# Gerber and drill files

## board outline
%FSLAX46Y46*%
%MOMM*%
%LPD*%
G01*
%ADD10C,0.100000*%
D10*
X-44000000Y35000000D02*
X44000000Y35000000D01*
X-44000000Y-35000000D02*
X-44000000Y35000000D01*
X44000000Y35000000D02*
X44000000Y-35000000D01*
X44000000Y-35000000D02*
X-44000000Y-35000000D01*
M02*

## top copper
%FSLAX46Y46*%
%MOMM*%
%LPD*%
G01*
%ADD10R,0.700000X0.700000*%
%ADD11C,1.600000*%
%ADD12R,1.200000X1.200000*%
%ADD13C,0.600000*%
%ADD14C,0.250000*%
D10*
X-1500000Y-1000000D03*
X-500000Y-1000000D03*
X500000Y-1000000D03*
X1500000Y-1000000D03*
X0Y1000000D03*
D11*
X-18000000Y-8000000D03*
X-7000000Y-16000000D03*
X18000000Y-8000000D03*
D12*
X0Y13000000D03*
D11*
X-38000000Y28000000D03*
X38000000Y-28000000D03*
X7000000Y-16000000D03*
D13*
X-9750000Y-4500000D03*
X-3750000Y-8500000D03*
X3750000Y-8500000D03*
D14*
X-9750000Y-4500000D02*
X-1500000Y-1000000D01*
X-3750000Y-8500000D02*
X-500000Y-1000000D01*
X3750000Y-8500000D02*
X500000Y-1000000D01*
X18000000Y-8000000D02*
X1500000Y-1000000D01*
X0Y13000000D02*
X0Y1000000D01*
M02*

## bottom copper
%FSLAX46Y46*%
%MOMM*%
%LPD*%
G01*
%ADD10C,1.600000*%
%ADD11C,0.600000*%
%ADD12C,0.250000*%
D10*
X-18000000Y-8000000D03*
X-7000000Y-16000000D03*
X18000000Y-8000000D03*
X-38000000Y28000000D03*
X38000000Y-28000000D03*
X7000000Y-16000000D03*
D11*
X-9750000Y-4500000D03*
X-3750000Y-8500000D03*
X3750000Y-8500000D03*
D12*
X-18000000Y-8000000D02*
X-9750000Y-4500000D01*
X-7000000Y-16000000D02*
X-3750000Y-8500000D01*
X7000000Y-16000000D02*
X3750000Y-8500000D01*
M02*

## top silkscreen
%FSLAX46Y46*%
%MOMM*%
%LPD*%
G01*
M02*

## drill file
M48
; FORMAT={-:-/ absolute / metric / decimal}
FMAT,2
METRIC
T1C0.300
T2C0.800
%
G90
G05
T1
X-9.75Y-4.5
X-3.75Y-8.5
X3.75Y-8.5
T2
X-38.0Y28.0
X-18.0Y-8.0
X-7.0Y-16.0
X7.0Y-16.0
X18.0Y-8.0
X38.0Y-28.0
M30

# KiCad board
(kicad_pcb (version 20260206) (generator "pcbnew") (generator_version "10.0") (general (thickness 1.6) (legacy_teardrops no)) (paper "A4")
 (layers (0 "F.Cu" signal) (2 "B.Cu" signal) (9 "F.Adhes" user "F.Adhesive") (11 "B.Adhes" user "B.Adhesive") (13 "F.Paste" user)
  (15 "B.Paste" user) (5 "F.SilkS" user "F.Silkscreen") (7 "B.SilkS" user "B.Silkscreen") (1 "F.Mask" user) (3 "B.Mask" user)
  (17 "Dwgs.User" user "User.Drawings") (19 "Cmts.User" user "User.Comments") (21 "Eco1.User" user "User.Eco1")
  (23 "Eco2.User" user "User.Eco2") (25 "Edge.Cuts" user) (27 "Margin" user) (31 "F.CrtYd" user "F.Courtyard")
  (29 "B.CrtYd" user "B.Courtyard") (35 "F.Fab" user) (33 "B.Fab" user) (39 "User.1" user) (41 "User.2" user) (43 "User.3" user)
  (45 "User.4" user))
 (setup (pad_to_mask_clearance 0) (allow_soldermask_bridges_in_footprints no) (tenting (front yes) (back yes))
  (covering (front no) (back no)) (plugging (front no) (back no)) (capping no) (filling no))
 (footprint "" (layer "F.Cu") (at 0 0)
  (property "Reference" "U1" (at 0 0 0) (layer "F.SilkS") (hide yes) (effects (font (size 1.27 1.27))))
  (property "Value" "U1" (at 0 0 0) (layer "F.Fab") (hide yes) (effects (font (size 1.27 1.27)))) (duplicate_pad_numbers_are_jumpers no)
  (pad "1" smd rect (at -1.5 1) (size 0.7 0.7) (layers "F.Cu" "F.Mask" "F.Paste") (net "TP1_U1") (thermal_bridge_angle 45))
  (pad "2" smd rect (at -0.5 1) (size 0.7 0.7) (layers "F.Cu" "F.Mask" "F.Paste") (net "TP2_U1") (thermal_bridge_angle 45))
  (pad "3" smd rect (at 0.5 1) (size 0.7 0.7) (layers "F.Cu" "F.Mask" "F.Paste") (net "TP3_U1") (thermal_bridge_angle 45))
  (pad "4" smd rect (at 1.5 1) (size 0.7 0.7) (layers "F.Cu" "F.Mask" "F.Paste") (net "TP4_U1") (thermal_bridge_angle 45))
  (pad "5" smd rect (at 0 -1) (size 0.7 0.7) (layers "F.Cu" "F.Mask" "F.Paste") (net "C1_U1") (thermal_bridge_angle 45)))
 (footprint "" (layer "F.Cu") (at -18 8)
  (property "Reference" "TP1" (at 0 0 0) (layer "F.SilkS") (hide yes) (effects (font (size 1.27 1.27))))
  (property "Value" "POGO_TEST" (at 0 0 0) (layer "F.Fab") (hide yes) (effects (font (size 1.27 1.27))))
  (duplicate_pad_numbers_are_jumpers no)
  (pad "1" thru_hole circle (at 0 0) (size 1.6 1.6) (drill 0.8) (layers "*.Cu" "*.Mask") (remove_unused_layers no) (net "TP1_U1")))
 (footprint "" (layer "F.Cu") (at -7 16)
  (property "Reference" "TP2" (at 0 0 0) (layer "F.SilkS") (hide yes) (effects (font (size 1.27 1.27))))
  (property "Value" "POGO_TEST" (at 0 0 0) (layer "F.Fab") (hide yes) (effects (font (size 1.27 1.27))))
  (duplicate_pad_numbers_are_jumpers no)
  (pad "1" thru_hole circle (at 0 0) (size 1.6 1.6) (drill 0.8) (layers "*.Cu" "*.Mask") (remove_unused_layers no) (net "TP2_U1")))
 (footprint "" (layer "F.Cu") (at 18 8)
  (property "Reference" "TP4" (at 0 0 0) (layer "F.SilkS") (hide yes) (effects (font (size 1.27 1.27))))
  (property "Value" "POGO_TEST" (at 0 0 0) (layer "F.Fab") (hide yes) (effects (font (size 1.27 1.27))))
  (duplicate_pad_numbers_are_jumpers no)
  (pad "1" thru_hole circle (at 0 0) (size 1.6 1.6) (drill 0.8) (layers "*.Cu" "*.Mask") (remove_unused_layers no) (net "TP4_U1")))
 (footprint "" (layer "F.Cu") (at 0 -13)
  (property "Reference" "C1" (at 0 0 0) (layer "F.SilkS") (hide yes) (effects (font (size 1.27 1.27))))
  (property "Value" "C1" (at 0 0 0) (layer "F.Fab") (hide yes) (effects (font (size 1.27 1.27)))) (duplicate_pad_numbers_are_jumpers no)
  (pad "1" smd rect (at 0 0) (size 1.2 1.2) (layers "F.Cu" "F.Mask" "F.Paste") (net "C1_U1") (thermal_bridge_angle 45)))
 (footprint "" (layer "F.Cu") (at -38 -28)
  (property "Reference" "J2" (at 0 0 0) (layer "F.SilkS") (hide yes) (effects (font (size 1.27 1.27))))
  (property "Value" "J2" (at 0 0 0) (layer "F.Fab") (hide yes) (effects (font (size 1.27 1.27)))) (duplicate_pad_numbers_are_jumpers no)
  (pad "1" thru_hole circle (at 0 0) (size 1.6 1.6) (drill 0.8) (layers "*.Cu" "*.Mask") (remove_unused_layers no) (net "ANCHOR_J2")))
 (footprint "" (layer "F.Cu") (at 38 28)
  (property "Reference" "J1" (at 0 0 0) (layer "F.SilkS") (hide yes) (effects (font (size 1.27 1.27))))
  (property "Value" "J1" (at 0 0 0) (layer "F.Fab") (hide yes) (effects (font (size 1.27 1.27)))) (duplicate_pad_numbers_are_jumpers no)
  (pad "1" thru_hole circle (at 0 0) (size 1.6 1.6) (drill 0.8) (layers "*.Cu" "*.Mask") (remove_unused_layers no) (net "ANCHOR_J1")))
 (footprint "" (layer "F.Cu") (at 7 16)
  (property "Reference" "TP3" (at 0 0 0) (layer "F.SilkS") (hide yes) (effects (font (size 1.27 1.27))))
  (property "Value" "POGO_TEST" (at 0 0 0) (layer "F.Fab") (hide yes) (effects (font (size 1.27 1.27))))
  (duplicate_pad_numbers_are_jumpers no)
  (pad "1" thru_hole circle (at 0 0) (size 1.6 1.6) (drill 0.8) (layers "*.Cu" "*.Mask") (remove_unused_layers no) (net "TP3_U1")))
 (gr_line (start -44 -35) (end 44 -35) (stroke (width 0.1) (type default)) (layer "Edge.Cuts"))
 (gr_line (start -44 35) (end -44 -35) (stroke (width 0.1) (type default)) (layer "Edge.Cuts"))
 (gr_line (start 44 -35) (end 44 35) (stroke (width 0.1) (type default)) (layer "Edge.Cuts"))
 (gr_line (start 44 35) (end -44 35) (stroke (width 0.1) (type default)) (layer "Edge.Cuts"))
 (segment (start -9.75 4.5) (end -1.5 1) (width 0.25) (layer "F.Cu") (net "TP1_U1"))
 (via (at -9.75 4.5) (size 0.6) (drill 0.3) (layers "F.Cu" "B.Cu") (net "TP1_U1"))
 (segment (start -18 8) (end -9.75 4.5) (width 0.25) (layer "B.Cu") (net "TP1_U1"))
 (segment (start -3.75 8.5) (end -0.5 1) (width 0.25) (layer "F.Cu") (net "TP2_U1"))
 (via (at -3.75 8.5) (size 0.6) (drill 0.3) (layers "F.Cu" "B.Cu") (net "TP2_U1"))
 (segment (start -7 16) (end -3.75 8.5) (width 0.25) (layer "B.Cu") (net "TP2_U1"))
 (segment (start 3.75 8.5) (end 0.5 1) (width 0.25) (layer "F.Cu") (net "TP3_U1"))
 (via (at 3.75 8.5) (size 0.6) (drill 0.3) (layers "F.Cu" "B.Cu") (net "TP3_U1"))
 (segment (start 7 16) (end 3.75 8.5) (width 0.25) (layer "B.Cu") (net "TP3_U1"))
 (segment (start 18 8) (end 1.5 1) (width 0.25) (layer "F.Cu") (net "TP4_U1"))
 (segment (start 0 -13) (end 0 -1) (width 0.25) (layer "F.Cu") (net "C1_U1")))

